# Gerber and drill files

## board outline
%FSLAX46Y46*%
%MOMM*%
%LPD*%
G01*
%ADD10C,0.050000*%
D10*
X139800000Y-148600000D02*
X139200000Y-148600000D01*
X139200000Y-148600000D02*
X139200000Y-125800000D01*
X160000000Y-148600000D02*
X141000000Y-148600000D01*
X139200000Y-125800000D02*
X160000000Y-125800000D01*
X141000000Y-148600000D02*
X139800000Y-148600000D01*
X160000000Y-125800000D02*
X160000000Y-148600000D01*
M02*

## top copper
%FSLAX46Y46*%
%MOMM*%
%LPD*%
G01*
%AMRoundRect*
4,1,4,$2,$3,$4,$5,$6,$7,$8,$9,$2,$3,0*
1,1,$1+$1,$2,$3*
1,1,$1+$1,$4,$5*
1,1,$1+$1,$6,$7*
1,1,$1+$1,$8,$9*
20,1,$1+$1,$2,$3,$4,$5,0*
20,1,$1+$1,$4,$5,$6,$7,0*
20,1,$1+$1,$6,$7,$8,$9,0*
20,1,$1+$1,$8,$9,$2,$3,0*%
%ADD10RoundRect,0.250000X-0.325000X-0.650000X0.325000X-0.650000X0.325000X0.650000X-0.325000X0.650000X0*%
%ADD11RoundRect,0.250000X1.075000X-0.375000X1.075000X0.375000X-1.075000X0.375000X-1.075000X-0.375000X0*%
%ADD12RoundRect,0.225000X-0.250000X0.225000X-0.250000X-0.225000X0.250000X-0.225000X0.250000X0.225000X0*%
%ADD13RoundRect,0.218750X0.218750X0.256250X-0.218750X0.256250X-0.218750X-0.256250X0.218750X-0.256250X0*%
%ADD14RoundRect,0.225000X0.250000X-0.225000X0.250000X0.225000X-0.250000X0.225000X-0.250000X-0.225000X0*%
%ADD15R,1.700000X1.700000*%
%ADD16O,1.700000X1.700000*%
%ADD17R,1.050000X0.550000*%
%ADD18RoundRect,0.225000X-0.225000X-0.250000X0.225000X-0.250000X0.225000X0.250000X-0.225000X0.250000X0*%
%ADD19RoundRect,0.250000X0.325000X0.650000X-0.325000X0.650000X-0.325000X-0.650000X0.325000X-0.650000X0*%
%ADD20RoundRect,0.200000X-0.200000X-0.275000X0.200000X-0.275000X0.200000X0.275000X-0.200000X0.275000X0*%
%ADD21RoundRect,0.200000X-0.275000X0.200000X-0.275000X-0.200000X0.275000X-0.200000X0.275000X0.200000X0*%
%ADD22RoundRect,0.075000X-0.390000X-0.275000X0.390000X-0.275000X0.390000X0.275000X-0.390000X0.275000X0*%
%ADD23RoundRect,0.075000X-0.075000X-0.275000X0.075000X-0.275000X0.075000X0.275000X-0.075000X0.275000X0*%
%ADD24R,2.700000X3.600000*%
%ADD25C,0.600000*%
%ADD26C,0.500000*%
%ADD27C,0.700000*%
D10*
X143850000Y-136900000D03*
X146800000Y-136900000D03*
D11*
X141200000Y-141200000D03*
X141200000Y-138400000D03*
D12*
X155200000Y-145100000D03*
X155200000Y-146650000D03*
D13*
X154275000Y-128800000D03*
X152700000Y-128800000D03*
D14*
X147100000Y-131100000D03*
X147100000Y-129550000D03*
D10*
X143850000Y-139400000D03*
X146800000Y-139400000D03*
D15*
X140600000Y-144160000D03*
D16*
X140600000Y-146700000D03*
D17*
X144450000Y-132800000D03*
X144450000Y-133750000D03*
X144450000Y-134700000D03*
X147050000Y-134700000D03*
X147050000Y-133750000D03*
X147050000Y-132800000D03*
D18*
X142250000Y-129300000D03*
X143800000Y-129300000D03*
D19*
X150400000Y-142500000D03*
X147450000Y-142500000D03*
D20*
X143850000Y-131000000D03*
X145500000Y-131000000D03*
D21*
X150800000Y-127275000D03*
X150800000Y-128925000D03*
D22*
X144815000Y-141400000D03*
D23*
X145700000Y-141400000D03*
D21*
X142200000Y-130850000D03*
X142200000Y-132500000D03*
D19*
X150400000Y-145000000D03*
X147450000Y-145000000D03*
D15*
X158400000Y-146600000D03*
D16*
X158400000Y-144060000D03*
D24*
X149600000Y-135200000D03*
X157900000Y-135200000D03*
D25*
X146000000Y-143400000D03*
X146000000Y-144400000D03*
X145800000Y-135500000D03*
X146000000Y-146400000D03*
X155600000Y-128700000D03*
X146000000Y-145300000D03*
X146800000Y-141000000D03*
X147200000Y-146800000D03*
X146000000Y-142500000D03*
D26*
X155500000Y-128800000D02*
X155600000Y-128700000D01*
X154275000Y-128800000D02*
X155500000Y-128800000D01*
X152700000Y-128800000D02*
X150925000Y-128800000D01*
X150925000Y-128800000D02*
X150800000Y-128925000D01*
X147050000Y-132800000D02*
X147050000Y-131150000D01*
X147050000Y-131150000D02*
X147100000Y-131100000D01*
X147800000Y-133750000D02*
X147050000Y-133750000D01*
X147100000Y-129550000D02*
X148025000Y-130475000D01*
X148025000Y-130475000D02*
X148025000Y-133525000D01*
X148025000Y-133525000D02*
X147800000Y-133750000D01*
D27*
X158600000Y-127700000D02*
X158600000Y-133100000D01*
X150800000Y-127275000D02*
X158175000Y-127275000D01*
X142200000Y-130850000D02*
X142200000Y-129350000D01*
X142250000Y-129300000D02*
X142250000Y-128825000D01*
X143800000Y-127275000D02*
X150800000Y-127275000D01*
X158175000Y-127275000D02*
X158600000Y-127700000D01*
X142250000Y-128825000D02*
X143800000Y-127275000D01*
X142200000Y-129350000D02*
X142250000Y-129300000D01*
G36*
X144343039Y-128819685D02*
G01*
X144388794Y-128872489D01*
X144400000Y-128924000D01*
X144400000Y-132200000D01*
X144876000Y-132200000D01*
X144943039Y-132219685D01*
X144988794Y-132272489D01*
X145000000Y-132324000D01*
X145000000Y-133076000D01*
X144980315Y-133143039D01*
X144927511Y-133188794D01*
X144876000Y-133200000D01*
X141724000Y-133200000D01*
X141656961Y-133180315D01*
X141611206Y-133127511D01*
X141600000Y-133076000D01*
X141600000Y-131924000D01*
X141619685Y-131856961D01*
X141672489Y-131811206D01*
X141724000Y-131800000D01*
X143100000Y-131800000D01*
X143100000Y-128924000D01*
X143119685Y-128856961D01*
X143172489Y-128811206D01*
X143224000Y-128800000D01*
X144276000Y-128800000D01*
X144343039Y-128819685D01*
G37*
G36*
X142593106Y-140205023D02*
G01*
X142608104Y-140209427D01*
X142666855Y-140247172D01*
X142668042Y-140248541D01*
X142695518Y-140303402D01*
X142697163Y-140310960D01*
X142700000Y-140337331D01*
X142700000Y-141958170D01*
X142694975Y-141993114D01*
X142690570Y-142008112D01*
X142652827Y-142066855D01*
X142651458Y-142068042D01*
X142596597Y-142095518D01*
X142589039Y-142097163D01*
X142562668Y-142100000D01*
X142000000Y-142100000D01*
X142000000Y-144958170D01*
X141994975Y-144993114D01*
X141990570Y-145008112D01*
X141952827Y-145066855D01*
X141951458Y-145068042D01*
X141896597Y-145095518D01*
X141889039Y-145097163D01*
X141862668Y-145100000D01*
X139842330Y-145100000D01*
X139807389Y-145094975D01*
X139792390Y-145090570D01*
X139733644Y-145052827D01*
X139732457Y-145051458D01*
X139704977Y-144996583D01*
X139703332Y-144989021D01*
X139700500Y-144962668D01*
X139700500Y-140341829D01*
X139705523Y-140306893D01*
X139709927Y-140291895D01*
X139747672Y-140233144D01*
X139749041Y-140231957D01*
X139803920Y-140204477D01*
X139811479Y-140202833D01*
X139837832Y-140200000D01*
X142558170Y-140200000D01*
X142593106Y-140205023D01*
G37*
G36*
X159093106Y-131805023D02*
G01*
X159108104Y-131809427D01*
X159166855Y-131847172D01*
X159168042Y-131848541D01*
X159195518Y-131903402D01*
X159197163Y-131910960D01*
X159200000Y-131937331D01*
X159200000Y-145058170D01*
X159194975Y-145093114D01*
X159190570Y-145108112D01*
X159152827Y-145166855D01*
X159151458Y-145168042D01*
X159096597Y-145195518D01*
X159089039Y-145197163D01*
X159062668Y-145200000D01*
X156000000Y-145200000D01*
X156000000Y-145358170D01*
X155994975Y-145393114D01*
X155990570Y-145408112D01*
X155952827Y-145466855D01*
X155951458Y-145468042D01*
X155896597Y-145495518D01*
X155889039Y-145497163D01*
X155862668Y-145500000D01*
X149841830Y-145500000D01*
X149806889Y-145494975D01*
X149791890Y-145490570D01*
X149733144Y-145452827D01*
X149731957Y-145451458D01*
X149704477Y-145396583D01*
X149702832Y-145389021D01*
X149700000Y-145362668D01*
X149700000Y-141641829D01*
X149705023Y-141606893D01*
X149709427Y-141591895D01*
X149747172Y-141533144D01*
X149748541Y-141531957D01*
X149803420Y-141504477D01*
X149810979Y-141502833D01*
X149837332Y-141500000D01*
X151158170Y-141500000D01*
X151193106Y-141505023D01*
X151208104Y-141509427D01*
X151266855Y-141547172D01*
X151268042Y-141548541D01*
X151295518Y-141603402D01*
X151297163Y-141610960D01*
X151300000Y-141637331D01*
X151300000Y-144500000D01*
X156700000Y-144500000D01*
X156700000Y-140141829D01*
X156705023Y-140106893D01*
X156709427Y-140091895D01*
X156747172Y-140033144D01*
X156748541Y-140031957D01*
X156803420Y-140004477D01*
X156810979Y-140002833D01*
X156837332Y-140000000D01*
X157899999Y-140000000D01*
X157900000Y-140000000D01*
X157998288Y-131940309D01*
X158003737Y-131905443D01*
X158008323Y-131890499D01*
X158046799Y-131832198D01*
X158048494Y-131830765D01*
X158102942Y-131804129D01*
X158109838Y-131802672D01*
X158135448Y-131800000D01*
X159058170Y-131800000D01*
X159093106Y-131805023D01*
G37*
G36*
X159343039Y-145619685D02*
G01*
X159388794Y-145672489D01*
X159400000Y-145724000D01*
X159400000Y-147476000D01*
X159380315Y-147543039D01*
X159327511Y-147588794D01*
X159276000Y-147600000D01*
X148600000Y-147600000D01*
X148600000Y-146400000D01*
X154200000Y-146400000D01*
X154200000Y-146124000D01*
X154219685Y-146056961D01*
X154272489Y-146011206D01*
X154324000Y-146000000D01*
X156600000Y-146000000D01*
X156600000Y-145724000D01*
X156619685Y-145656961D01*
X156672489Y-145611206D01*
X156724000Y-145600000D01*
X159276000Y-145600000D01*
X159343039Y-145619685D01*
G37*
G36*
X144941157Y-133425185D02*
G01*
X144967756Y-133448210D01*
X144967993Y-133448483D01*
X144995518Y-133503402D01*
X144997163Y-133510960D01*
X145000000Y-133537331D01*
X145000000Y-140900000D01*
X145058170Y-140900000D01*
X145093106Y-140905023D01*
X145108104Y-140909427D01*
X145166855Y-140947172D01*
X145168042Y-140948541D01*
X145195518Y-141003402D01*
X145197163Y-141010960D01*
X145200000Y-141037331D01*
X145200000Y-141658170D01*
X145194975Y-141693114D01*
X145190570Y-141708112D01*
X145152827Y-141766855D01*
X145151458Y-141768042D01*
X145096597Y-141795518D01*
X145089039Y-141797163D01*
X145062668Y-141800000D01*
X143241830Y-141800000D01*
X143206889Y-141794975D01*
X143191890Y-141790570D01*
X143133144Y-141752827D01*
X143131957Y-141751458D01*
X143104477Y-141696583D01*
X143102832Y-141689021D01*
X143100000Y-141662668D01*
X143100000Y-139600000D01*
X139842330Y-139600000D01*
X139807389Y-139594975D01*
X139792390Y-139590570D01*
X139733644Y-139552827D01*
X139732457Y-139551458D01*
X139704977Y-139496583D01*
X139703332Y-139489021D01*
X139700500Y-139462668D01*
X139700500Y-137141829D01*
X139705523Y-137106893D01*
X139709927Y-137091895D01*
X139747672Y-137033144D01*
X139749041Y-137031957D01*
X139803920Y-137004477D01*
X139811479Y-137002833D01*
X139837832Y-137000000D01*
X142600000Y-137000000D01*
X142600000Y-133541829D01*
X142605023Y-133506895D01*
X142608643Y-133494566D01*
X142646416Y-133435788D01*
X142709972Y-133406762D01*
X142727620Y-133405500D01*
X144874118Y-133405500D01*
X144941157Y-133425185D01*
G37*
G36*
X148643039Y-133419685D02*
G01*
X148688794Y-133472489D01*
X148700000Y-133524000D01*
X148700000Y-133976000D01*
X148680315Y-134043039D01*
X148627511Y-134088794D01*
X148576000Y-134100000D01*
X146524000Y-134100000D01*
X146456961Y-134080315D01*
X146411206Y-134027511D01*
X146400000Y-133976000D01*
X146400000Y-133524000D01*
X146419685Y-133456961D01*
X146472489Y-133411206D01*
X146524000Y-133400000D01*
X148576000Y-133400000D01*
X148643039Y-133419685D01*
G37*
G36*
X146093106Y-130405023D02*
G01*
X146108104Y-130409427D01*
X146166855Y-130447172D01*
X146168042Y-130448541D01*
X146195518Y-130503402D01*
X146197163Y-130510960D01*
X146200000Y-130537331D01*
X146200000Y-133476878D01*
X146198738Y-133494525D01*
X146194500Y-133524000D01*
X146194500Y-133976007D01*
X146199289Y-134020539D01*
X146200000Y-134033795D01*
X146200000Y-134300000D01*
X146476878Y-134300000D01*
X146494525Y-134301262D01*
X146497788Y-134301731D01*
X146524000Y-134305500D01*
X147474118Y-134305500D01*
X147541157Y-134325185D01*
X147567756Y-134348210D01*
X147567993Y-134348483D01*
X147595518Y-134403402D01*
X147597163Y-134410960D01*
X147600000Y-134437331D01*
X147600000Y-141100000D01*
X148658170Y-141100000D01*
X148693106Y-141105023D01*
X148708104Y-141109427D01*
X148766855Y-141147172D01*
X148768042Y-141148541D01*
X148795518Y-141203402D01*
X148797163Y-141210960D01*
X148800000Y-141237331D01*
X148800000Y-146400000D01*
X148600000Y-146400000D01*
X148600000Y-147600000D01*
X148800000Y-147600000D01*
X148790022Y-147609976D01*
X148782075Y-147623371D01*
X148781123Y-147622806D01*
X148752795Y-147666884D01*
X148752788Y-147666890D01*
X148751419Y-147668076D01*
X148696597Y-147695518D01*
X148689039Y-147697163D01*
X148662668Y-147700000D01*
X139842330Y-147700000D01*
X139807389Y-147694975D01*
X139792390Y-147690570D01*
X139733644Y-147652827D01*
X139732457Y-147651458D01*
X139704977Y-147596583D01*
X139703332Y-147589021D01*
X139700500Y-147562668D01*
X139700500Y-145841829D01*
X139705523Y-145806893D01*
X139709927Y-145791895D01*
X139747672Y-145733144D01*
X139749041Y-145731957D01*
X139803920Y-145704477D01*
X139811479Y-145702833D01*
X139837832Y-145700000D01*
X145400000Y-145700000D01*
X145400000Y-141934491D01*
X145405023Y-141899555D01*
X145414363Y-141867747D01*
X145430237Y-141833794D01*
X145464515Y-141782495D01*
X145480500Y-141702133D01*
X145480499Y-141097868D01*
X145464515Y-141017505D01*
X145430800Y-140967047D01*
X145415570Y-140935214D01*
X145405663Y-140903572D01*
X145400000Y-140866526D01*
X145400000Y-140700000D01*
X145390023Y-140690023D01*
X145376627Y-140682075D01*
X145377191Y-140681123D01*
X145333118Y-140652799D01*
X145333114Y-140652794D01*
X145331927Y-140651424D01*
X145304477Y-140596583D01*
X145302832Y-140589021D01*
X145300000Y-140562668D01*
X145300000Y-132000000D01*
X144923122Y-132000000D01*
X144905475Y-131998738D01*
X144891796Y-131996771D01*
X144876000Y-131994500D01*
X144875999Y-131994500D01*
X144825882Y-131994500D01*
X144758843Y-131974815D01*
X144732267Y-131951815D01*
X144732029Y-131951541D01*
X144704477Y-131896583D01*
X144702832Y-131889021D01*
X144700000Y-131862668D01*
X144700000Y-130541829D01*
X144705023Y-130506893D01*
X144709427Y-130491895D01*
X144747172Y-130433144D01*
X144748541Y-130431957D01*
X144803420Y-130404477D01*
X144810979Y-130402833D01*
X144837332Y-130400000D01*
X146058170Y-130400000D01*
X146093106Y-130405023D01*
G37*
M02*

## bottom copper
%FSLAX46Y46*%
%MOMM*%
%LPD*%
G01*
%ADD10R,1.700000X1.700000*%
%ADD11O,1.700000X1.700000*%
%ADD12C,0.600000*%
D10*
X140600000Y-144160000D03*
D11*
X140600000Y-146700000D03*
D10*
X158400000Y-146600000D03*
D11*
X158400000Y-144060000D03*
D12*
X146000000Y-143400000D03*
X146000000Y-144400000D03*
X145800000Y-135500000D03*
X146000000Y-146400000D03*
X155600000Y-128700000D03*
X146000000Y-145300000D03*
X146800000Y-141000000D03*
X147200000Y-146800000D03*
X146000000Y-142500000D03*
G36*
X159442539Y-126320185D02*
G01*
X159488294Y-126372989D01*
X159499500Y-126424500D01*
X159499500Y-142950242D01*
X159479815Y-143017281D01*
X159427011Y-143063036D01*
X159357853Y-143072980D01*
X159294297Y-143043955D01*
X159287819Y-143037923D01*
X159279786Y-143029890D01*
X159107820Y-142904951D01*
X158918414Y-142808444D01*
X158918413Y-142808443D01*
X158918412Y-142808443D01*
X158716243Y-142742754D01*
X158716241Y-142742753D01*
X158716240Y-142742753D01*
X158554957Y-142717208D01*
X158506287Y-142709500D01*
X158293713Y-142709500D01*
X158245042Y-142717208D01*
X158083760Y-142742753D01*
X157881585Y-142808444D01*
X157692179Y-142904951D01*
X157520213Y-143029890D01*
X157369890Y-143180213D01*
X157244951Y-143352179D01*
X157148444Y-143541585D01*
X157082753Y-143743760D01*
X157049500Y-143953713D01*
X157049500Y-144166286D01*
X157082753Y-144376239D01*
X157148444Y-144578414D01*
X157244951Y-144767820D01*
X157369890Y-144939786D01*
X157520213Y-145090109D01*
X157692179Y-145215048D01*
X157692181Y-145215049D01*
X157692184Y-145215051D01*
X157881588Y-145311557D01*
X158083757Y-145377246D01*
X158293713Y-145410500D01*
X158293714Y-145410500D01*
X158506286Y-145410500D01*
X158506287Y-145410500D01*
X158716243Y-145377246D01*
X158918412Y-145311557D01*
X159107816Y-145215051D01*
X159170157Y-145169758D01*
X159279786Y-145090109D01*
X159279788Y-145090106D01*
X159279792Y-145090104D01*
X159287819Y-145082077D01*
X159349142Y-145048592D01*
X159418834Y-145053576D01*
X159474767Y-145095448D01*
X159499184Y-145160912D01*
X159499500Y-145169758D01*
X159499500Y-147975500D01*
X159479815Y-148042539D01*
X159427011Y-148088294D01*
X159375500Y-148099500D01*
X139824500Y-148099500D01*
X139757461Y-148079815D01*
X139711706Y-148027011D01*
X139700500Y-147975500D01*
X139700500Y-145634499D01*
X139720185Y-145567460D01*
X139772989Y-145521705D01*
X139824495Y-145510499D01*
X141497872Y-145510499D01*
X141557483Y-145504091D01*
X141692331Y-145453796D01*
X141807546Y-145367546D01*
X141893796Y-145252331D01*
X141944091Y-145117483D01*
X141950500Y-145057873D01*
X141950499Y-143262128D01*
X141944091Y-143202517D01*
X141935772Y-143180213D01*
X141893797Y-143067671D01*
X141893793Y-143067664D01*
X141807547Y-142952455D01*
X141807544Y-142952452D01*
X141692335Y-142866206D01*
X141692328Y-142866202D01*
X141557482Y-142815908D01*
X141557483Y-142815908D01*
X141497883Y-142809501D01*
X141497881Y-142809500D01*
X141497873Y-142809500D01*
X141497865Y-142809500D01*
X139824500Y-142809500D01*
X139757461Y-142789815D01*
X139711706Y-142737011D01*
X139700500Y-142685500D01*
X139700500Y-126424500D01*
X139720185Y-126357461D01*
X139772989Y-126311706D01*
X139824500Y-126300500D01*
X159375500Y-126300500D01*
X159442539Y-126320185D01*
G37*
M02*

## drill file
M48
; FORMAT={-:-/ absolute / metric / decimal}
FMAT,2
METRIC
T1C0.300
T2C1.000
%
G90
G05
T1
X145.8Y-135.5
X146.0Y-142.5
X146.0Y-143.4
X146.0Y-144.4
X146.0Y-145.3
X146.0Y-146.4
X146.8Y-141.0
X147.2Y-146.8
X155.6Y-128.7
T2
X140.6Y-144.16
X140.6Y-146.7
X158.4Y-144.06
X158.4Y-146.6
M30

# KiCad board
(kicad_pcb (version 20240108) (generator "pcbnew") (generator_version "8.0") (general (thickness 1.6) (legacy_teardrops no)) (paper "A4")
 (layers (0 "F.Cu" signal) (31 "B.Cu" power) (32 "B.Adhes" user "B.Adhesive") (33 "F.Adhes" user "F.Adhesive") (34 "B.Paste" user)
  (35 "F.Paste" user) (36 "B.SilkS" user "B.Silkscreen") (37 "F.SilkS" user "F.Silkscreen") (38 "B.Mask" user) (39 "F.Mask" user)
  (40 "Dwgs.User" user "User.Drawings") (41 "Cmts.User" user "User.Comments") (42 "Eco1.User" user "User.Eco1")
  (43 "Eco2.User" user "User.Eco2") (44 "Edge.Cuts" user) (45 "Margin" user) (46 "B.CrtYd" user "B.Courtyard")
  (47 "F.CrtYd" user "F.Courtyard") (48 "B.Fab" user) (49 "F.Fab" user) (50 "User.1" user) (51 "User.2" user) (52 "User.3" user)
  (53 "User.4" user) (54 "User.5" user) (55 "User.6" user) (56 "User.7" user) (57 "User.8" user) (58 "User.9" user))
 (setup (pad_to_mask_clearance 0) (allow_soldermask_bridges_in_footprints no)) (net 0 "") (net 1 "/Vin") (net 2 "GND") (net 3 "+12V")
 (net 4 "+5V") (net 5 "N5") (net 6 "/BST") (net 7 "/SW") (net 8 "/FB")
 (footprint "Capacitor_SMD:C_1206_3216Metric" (layer "F.Cu") (at 145.325 136.9)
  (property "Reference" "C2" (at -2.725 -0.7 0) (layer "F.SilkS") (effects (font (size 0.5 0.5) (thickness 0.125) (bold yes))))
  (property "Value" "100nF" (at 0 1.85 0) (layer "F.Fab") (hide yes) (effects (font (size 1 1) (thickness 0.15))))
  (pad "1" smd roundrect (at -1.475 0) (size 1.15 1.8) (layers "F.Cu" "F.Paste" "F.Mask") (roundrect_rratio 0.217391) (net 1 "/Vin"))
  (pad "2" smd roundrect (at 1.475 0) (size 1.15 1.8) (layers "F.Cu" "F.Paste" "F.Mask") (roundrect_rratio 0.217391) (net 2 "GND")))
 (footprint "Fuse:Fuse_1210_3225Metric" (layer "F.Cu") (at 141.2 139.8 90)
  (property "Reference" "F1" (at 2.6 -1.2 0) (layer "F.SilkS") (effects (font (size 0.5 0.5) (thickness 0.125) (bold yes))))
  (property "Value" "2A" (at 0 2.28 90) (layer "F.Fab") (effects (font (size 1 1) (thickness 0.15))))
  (pad "1" smd roundrect (at -1.4 0 90) (size 1.25 2.65) (layers "F.Cu" "F.Paste" "F.Mask") (roundrect_rratio 0.2) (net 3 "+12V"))
  (pad "2" smd roundrect (at 1.4 0 90) (size 1.25 2.65) (layers "F.Cu" "F.Paste" "F.Mask") (roundrect_rratio 0.2) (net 1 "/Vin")))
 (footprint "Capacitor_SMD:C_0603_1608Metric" (layer "F.Cu") (at 155.2 145.875 -90)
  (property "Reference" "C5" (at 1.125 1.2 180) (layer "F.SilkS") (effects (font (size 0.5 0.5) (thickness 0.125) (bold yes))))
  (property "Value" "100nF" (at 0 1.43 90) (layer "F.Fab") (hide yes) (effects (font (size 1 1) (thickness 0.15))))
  (pad "1" smd roundrect (at -0.775 0 270) (size 0.9 0.95) (layers "F.Cu" "F.Paste" "F.Mask") (roundrect_rratio 0.25) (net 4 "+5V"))
  (pad "2" smd roundrect (at 0.775 0 270) (size 0.9 0.95) (layers "F.Cu" "F.Paste" "F.Mask") (roundrect_rratio 0.25) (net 2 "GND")))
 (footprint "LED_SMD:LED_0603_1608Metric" (layer "F.Cu") (at 153.4875 128.8 180)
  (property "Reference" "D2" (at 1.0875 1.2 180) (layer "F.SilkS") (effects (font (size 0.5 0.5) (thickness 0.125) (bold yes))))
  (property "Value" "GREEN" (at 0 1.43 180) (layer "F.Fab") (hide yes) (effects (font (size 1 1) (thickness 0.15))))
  (pad "1" smd roundrect (at -0.7875 0 180) (size 0.875 0.95) (layers "F.Cu" "F.Paste" "F.Mask") (roundrect_rratio 0.25) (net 2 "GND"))
  (pad "2" smd roundrect (at 0.7875 0 180) (size 0.875 0.95) (layers "F.Cu" "F.Paste" "F.Mask") (roundrect_rratio 0.25) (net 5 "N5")))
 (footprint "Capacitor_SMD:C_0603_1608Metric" (layer "F.Cu") (at 147.1 130.325 90)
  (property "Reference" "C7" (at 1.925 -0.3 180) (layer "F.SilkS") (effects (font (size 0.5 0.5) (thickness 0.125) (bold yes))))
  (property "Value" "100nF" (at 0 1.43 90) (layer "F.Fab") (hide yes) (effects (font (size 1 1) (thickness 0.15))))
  (pad "1" smd roundrect (at -0.775 0 90) (size 0.9 0.95) (layers "F.Cu" "F.Paste" "F.Mask") (roundrect_rratio 0.25) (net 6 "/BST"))
  (pad "2" smd roundrect (at 0.775 0 90) (size 0.9 0.95) (layers "F.Cu" "F.Paste" "F.Mask") (roundrect_rratio 0.25) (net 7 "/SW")))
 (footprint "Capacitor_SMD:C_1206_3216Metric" (layer "F.Cu") (at 145.325 139.4)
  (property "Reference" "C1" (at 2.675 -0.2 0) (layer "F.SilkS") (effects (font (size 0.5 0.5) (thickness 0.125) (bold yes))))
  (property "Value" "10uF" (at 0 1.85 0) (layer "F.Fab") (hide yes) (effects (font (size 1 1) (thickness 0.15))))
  (pad "1" smd roundrect (at -1.475 0) (size 1.15 1.8) (layers "F.Cu" "F.Paste" "F.Mask") (roundrect_rratio 0.217391) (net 1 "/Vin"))
  (pad "2" smd roundrect (at 1.475 0) (size 1.15 1.8) (layers "F.Cu" "F.Paste" "F.Mask") (roundrect_rratio 0.217391) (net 2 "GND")))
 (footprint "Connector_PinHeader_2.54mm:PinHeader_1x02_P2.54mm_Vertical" (layer "F.Cu") (at 140.6 144.16)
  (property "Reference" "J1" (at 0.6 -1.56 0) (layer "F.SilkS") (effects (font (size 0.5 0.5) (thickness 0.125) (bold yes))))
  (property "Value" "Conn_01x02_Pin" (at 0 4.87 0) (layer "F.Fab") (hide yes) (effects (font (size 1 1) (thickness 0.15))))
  (pad "1" thru_hole rect (at 0 0) (size 1.7 1.7) (drill 1) (layers "*.Cu" "*.Mask") (remove_unused_layers no) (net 3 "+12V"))
  (pad "2" thru_hole oval (at 0 2.54) (size 1.7 1.7) (drill 1) (layers "*.Cu" "*.Mask") (remove_unused_layers no) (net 2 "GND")))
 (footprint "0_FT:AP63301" (layer "F.Cu") (at 145.75 133.75)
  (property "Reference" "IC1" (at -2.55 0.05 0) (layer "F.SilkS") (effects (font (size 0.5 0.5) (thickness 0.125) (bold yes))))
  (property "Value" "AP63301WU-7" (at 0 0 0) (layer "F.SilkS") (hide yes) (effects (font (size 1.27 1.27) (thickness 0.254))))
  (pad "1" smd rect (at -1.3 -0.95 90) (size 0.55 1.05) (layers "F.Cu" "F.Paste" "F.Mask") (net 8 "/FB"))
  (pad "2" smd rect (at -1.3 0 90) (size 0.55 1.05) (layers "F.Cu" "F.Paste" "F.Mask") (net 1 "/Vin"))
  (pad "3" smd rect (at -1.3 0.95 90) (size 0.55 1.05) (layers "F.Cu" "F.Paste" "F.Mask") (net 1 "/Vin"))
  (pad "4" smd rect (at 1.3 0.95 90) (size 0.55 1.05) (layers "F.Cu" "F.Paste" "F.Mask") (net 2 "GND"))
  (pad "5" smd rect (at 1.3 0 90) (size 0.55 1.05) (layers "F.Cu" "F.Paste" "F.Mask") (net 7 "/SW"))
  (pad "6" smd rect (at 1.3 -0.95 90) (size 0.55 1.05) (layers "F.Cu" "F.Paste" "F.Mask") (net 6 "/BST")))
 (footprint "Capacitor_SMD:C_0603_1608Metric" (layer "F.Cu") (at 143.025 129.3)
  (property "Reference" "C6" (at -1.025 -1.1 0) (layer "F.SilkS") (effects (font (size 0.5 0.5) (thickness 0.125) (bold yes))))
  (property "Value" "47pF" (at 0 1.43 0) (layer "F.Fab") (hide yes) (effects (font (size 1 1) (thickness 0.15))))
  (pad "1" smd roundrect (at -0.775 0) (size 0.9 0.95) (layers "F.Cu" "F.Paste" "F.Mask") (roundrect_rratio 0.25) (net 4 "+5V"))
  (pad "2" smd roundrect (at 0.775 0) (size 0.9 0.95) (layers "F.Cu" "F.Paste" "F.Mask") (roundrect_rratio 0.25) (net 8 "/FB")))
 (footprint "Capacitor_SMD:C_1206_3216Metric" (layer "F.Cu") (at 148.925 142.5 180)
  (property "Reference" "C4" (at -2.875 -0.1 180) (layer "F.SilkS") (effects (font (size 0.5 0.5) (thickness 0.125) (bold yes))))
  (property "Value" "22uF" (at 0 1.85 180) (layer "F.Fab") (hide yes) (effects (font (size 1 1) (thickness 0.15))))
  (pad "1" smd roundrect (at -1.475 0 180) (size 1.15 1.8) (layers "F.Cu" "F.Paste" "F.Mask") (roundrect_rratio 0.217391) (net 4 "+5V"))
  (pad "2" smd roundrect (at 1.475 0 180) (size 1.15 1.8) (layers "F.Cu" "F.Paste" "F.Mask") (roundrect_rratio 0.217391) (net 2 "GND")))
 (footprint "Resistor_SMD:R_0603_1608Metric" (layer "F.Cu") (at 144.675 131)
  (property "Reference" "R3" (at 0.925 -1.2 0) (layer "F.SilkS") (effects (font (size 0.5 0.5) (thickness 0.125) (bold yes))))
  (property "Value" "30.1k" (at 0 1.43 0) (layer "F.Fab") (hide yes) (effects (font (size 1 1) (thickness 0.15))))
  (pad "1" smd roundrect (at -0.825 0) (size 0.8 0.95) (layers "F.Cu" "F.Paste" "F.Mask") (roundrect_rratio 0.25) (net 8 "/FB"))
  (pad "2" smd roundrect (at 0.825 0) (size 0.8 0.95) (layers "F.Cu" "F.Paste" "F.Mask") (roundrect_rratio 0.25) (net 2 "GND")))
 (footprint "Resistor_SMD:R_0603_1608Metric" (layer "F.Cu") (at 150.8 128.1 -90)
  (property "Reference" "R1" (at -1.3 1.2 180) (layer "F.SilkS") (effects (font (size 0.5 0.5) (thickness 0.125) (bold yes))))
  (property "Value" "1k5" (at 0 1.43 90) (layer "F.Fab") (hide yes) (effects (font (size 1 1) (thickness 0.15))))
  (pad "1" smd roundrect (at -0.825 0 270) (size 0.8 0.95) (layers "F.Cu" "F.Paste" "F.Mask") (roundrect_rratio 0.25) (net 4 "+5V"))
  (pad "2" smd roundrect (at 0.825 0 270) (size 0.8 0.95) (layers "F.Cu" "F.Paste" "F.Mask") (roundrect_rratio 0.25) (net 5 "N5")))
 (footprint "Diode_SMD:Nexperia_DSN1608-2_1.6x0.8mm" (layer "F.Cu") (at 145.1 141.4)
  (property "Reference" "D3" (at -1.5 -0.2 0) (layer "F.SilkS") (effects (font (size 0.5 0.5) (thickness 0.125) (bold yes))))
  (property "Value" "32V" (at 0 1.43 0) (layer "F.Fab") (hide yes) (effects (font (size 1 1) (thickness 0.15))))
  (pad "1" smd roundrect (at -0.285 0) (size 0.93 0.7) (layers "F.Cu" "F.Paste" "F.Mask") (roundrect_rratio 0.1071428571) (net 1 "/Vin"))
  (pad "2" smd roundrect (at 0.6 0) (size 0.3 0.7) (layers "F.Cu" "F.Paste" "F.Mask") (roundrect_rratio 0.25) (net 2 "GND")))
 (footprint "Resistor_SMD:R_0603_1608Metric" (layer "F.Cu") (at 142.2 131.675 -90)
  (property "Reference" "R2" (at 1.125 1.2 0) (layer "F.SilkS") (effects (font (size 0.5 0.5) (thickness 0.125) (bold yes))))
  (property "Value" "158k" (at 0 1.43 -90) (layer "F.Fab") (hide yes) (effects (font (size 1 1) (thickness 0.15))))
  (pad "1" smd roundrect (at -0.825 0 270) (size 0.8 0.95) (layers "F.Cu" "F.Paste" "F.Mask") (roundrect_rratio 0.25) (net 4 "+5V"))
  (pad "2" smd roundrect (at 0.825 0 270) (size 0.8 0.95) (layers "F.Cu" "F.Paste" "F.Mask") (roundrect_rratio 0.25) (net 8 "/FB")))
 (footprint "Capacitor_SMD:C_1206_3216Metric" (layer "F.Cu") (at 148.925 145 180)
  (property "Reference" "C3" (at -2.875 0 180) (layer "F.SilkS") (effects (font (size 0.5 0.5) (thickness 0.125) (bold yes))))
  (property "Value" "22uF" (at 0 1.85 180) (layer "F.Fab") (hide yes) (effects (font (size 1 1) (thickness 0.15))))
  (pad "1" smd roundrect (at -1.475 0 180) (size 1.15 1.8) (layers "F.Cu" "F.Paste" "F.Mask") (roundrect_rratio 0.217391) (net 4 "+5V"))
  (pad "2" smd roundrect (at 1.475 0 180) (size 1.15 1.8) (layers "F.Cu" "F.Paste" "F.Mask") (roundrect_rratio 0.217391) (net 2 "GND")))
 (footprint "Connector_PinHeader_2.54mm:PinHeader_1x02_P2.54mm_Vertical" (layer "F.Cu") (at 158.4 146.6 180)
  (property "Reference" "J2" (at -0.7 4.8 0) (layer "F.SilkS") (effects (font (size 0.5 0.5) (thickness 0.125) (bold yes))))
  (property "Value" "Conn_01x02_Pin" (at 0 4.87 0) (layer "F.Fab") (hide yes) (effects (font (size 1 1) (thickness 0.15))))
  (pad "1" thru_hole rect (at 0 0 180) (size 1.7 1.7) (drill 1) (layers "*.Cu" "*.Mask") (remove_unused_layers no) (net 2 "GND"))
  (pad "2" thru_hole oval (at 0 2.54 180) (size 1.7 1.7) (drill 1) (layers "*.Cu" "*.Mask") (remove_unused_layers no) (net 4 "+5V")))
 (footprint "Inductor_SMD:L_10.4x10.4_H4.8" (layer "F.Cu") (at 153.75 135.2)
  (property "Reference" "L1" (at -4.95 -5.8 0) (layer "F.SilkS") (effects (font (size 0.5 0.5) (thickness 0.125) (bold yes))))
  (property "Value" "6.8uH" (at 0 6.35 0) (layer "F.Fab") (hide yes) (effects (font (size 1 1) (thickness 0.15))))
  (pad "1" smd rect (at -4.15 0) (size 2.7 3.6) (layers "F.Cu" "F.Paste" "F.Mask") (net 7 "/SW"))
  (pad "2" smd rect (at 4.15 0) (size 2.7 3.6) (layers "F.Cu" "F.Paste" "F.Mask") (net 4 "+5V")))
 (gr_line (start 139.8 148.6) (end 139.2 148.6) (stroke (width 0.05) (type default)) (layer "Edge.Cuts"))
 (gr_line (start 139.2 148.6) (end 139.2 125.8) (stroke (width 0.05) (type default)) (layer "Edge.Cuts"))
 (gr_line (start 160 148.6) (end 141 148.6) (stroke (width 0.05) (type default)) (layer "Edge.Cuts"))
 (gr_line (start 139.2 125.8) (end 160 125.8) (stroke (width 0.05) (type default)) (layer "Edge.Cuts"))
 (gr_line (start 141 148.6) (end 139.8 148.6) (stroke (width 0.05) (type default)) (layer "Edge.Cuts"))
 (gr_line (start 160 125.8) (end 160 148.6) (stroke (width 0.05) (type default)) (layer "Edge.Cuts"))
 (segment (start 155.5 128.8) (end 155.6 128.7) (width 0.5) (layer "F.Cu") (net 2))
 (segment (start 154.275 128.8) (end 155.5 128.8) (width 0.5) (layer "F.Cu") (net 2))
 (via (at 146 143.4) (size 0.6) (drill 0.3) (layers "F.Cu" "B.Cu") (free yes) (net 2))
 (via (at 146 144.4) (size 0.6) (drill 0.3) (layers "F.Cu" "B.Cu") (free yes) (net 2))
 (via (at 145.8 135.5) (size 0.6) (drill 0.3) (layers "F.Cu" "B.Cu") (free yes) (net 2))
 (via (at 146 146.4) (size 0.6) (drill 0.3) (layers "F.Cu" "B.Cu") (free yes) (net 2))
 (via (at 155.6 128.7) (size 0.6) (drill 0.3) (layers "F.Cu" "B.Cu") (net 2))
 (via (at 146 145.3) (size 0.6) (drill 0.3) (layers "F.Cu" "B.Cu") (free yes) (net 2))
 (via (at 146.8 141) (size 0.6) (drill 0.3) (layers "F.Cu" "B.Cu") (free yes) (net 2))
 (via (at 147.2 146.8) (size 0.6) (drill 0.3) (layers "F.Cu" "B.Cu") (free yes) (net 2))
 (via (at 146 142.5) (size 0.6) (drill 0.3) (layers "F.Cu" "B.Cu") (free yes) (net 2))
 (segment (start 152.7 128.8) (end 150.925 128.8) (width 0.5) (layer "F.Cu") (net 5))
 (segment (start 150.925 128.8) (end 150.8 128.925) (width 0.5) (layer "F.Cu") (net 5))
 (segment (start 147.05 132.8) (end 147.05 131.15) (width 0.5) (layer "F.Cu") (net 6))
 (segment (start 147.05 131.15) (end 147.1 131.1) (width 0.5) (layer "F.Cu") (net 6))
 (segment (start 147.8 133.75) (end 147.05 133.75) (width 0.5) (layer "F.Cu") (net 7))
 (segment (start 147.1 129.55) (end 148.025 130.475) (width 0.5) (layer "F.Cu") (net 7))
 (segment (start 148.025 130.475) (end 148.025 133.525) (width 0.5) (layer "F.Cu") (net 7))
 (segment (start 148.025 133.525) (end 147.8 133.75) (width 0.5) (layer "F.Cu") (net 7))
 (segment (start 158.6 127.7) (end 158.6 133.1) (width 0.7) (layer "F.Cu") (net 4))
 (segment (start 150.8 127.275) (end 158.175 127.275) (width 0.7) (layer "F.Cu") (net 4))
 (segment (start 142.2 130.85) (end 142.2 129.35) (width 0.7) (layer "F.Cu") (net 4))
 (segment (start 142.25 129.3) (end 142.25 128.825) (width 0.7) (layer "F.Cu") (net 4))
 (segment (start 143.8 127.275) (end 150.8 127.275) (width 0.7) (layer "F.Cu") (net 4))
 (segment (start 158.175 127.275) (end 158.6 127.7) (width 0.7) (layer "F.Cu") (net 4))
 (segment (start 142.25 128.825) (end 143.8 127.275) (width 0.7) (layer "F.Cu") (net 4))
 (segment (start 142.2 129.35) (end 142.25 129.3) (width 0.7) (layer "F.Cu") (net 4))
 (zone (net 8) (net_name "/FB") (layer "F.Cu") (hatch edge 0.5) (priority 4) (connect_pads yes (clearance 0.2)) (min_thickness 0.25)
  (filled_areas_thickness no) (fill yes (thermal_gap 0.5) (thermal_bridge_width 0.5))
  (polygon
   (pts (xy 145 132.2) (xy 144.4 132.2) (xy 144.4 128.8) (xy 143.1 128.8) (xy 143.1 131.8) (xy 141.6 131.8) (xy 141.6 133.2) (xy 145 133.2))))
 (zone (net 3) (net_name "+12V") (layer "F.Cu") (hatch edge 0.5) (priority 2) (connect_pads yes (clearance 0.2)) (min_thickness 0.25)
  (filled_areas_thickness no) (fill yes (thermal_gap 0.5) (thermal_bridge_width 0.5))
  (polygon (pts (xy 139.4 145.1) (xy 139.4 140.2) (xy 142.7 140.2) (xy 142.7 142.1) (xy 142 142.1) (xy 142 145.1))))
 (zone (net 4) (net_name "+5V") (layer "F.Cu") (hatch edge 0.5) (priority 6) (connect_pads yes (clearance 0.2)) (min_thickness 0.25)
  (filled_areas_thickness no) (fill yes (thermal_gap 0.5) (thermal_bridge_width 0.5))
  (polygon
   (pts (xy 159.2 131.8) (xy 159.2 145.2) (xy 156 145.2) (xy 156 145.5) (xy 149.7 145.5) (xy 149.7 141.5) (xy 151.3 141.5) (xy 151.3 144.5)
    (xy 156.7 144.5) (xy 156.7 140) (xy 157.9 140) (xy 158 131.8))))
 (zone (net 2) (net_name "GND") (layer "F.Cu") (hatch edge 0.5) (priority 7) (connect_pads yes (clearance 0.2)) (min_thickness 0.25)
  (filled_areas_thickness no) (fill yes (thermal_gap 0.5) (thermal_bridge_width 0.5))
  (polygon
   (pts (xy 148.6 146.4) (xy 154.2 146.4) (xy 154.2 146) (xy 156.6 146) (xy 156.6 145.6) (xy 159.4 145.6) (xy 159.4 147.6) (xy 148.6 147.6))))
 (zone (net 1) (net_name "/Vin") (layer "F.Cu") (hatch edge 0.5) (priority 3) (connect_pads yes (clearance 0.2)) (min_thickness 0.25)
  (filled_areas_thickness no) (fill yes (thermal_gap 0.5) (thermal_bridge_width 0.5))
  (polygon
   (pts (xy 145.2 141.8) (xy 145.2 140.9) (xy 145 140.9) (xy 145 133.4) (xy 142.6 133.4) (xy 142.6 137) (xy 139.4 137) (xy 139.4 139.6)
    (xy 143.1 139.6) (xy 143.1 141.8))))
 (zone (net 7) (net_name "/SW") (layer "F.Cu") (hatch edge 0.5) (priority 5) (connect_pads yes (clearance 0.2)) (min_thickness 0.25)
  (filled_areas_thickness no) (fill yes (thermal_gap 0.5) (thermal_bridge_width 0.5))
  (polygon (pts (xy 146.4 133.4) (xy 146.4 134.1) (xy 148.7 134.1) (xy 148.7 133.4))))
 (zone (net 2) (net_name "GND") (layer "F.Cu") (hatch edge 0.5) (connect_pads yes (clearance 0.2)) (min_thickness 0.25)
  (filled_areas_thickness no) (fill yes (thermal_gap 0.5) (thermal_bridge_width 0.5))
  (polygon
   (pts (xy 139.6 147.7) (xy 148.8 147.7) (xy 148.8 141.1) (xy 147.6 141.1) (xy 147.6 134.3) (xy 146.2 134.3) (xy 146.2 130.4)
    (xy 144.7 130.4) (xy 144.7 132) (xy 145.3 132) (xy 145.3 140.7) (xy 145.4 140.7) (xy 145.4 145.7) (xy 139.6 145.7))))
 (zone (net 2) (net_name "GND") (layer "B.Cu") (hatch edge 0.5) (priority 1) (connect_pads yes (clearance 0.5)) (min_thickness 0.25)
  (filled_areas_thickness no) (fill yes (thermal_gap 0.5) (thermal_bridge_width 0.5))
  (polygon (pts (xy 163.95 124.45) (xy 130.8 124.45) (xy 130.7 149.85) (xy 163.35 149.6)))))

